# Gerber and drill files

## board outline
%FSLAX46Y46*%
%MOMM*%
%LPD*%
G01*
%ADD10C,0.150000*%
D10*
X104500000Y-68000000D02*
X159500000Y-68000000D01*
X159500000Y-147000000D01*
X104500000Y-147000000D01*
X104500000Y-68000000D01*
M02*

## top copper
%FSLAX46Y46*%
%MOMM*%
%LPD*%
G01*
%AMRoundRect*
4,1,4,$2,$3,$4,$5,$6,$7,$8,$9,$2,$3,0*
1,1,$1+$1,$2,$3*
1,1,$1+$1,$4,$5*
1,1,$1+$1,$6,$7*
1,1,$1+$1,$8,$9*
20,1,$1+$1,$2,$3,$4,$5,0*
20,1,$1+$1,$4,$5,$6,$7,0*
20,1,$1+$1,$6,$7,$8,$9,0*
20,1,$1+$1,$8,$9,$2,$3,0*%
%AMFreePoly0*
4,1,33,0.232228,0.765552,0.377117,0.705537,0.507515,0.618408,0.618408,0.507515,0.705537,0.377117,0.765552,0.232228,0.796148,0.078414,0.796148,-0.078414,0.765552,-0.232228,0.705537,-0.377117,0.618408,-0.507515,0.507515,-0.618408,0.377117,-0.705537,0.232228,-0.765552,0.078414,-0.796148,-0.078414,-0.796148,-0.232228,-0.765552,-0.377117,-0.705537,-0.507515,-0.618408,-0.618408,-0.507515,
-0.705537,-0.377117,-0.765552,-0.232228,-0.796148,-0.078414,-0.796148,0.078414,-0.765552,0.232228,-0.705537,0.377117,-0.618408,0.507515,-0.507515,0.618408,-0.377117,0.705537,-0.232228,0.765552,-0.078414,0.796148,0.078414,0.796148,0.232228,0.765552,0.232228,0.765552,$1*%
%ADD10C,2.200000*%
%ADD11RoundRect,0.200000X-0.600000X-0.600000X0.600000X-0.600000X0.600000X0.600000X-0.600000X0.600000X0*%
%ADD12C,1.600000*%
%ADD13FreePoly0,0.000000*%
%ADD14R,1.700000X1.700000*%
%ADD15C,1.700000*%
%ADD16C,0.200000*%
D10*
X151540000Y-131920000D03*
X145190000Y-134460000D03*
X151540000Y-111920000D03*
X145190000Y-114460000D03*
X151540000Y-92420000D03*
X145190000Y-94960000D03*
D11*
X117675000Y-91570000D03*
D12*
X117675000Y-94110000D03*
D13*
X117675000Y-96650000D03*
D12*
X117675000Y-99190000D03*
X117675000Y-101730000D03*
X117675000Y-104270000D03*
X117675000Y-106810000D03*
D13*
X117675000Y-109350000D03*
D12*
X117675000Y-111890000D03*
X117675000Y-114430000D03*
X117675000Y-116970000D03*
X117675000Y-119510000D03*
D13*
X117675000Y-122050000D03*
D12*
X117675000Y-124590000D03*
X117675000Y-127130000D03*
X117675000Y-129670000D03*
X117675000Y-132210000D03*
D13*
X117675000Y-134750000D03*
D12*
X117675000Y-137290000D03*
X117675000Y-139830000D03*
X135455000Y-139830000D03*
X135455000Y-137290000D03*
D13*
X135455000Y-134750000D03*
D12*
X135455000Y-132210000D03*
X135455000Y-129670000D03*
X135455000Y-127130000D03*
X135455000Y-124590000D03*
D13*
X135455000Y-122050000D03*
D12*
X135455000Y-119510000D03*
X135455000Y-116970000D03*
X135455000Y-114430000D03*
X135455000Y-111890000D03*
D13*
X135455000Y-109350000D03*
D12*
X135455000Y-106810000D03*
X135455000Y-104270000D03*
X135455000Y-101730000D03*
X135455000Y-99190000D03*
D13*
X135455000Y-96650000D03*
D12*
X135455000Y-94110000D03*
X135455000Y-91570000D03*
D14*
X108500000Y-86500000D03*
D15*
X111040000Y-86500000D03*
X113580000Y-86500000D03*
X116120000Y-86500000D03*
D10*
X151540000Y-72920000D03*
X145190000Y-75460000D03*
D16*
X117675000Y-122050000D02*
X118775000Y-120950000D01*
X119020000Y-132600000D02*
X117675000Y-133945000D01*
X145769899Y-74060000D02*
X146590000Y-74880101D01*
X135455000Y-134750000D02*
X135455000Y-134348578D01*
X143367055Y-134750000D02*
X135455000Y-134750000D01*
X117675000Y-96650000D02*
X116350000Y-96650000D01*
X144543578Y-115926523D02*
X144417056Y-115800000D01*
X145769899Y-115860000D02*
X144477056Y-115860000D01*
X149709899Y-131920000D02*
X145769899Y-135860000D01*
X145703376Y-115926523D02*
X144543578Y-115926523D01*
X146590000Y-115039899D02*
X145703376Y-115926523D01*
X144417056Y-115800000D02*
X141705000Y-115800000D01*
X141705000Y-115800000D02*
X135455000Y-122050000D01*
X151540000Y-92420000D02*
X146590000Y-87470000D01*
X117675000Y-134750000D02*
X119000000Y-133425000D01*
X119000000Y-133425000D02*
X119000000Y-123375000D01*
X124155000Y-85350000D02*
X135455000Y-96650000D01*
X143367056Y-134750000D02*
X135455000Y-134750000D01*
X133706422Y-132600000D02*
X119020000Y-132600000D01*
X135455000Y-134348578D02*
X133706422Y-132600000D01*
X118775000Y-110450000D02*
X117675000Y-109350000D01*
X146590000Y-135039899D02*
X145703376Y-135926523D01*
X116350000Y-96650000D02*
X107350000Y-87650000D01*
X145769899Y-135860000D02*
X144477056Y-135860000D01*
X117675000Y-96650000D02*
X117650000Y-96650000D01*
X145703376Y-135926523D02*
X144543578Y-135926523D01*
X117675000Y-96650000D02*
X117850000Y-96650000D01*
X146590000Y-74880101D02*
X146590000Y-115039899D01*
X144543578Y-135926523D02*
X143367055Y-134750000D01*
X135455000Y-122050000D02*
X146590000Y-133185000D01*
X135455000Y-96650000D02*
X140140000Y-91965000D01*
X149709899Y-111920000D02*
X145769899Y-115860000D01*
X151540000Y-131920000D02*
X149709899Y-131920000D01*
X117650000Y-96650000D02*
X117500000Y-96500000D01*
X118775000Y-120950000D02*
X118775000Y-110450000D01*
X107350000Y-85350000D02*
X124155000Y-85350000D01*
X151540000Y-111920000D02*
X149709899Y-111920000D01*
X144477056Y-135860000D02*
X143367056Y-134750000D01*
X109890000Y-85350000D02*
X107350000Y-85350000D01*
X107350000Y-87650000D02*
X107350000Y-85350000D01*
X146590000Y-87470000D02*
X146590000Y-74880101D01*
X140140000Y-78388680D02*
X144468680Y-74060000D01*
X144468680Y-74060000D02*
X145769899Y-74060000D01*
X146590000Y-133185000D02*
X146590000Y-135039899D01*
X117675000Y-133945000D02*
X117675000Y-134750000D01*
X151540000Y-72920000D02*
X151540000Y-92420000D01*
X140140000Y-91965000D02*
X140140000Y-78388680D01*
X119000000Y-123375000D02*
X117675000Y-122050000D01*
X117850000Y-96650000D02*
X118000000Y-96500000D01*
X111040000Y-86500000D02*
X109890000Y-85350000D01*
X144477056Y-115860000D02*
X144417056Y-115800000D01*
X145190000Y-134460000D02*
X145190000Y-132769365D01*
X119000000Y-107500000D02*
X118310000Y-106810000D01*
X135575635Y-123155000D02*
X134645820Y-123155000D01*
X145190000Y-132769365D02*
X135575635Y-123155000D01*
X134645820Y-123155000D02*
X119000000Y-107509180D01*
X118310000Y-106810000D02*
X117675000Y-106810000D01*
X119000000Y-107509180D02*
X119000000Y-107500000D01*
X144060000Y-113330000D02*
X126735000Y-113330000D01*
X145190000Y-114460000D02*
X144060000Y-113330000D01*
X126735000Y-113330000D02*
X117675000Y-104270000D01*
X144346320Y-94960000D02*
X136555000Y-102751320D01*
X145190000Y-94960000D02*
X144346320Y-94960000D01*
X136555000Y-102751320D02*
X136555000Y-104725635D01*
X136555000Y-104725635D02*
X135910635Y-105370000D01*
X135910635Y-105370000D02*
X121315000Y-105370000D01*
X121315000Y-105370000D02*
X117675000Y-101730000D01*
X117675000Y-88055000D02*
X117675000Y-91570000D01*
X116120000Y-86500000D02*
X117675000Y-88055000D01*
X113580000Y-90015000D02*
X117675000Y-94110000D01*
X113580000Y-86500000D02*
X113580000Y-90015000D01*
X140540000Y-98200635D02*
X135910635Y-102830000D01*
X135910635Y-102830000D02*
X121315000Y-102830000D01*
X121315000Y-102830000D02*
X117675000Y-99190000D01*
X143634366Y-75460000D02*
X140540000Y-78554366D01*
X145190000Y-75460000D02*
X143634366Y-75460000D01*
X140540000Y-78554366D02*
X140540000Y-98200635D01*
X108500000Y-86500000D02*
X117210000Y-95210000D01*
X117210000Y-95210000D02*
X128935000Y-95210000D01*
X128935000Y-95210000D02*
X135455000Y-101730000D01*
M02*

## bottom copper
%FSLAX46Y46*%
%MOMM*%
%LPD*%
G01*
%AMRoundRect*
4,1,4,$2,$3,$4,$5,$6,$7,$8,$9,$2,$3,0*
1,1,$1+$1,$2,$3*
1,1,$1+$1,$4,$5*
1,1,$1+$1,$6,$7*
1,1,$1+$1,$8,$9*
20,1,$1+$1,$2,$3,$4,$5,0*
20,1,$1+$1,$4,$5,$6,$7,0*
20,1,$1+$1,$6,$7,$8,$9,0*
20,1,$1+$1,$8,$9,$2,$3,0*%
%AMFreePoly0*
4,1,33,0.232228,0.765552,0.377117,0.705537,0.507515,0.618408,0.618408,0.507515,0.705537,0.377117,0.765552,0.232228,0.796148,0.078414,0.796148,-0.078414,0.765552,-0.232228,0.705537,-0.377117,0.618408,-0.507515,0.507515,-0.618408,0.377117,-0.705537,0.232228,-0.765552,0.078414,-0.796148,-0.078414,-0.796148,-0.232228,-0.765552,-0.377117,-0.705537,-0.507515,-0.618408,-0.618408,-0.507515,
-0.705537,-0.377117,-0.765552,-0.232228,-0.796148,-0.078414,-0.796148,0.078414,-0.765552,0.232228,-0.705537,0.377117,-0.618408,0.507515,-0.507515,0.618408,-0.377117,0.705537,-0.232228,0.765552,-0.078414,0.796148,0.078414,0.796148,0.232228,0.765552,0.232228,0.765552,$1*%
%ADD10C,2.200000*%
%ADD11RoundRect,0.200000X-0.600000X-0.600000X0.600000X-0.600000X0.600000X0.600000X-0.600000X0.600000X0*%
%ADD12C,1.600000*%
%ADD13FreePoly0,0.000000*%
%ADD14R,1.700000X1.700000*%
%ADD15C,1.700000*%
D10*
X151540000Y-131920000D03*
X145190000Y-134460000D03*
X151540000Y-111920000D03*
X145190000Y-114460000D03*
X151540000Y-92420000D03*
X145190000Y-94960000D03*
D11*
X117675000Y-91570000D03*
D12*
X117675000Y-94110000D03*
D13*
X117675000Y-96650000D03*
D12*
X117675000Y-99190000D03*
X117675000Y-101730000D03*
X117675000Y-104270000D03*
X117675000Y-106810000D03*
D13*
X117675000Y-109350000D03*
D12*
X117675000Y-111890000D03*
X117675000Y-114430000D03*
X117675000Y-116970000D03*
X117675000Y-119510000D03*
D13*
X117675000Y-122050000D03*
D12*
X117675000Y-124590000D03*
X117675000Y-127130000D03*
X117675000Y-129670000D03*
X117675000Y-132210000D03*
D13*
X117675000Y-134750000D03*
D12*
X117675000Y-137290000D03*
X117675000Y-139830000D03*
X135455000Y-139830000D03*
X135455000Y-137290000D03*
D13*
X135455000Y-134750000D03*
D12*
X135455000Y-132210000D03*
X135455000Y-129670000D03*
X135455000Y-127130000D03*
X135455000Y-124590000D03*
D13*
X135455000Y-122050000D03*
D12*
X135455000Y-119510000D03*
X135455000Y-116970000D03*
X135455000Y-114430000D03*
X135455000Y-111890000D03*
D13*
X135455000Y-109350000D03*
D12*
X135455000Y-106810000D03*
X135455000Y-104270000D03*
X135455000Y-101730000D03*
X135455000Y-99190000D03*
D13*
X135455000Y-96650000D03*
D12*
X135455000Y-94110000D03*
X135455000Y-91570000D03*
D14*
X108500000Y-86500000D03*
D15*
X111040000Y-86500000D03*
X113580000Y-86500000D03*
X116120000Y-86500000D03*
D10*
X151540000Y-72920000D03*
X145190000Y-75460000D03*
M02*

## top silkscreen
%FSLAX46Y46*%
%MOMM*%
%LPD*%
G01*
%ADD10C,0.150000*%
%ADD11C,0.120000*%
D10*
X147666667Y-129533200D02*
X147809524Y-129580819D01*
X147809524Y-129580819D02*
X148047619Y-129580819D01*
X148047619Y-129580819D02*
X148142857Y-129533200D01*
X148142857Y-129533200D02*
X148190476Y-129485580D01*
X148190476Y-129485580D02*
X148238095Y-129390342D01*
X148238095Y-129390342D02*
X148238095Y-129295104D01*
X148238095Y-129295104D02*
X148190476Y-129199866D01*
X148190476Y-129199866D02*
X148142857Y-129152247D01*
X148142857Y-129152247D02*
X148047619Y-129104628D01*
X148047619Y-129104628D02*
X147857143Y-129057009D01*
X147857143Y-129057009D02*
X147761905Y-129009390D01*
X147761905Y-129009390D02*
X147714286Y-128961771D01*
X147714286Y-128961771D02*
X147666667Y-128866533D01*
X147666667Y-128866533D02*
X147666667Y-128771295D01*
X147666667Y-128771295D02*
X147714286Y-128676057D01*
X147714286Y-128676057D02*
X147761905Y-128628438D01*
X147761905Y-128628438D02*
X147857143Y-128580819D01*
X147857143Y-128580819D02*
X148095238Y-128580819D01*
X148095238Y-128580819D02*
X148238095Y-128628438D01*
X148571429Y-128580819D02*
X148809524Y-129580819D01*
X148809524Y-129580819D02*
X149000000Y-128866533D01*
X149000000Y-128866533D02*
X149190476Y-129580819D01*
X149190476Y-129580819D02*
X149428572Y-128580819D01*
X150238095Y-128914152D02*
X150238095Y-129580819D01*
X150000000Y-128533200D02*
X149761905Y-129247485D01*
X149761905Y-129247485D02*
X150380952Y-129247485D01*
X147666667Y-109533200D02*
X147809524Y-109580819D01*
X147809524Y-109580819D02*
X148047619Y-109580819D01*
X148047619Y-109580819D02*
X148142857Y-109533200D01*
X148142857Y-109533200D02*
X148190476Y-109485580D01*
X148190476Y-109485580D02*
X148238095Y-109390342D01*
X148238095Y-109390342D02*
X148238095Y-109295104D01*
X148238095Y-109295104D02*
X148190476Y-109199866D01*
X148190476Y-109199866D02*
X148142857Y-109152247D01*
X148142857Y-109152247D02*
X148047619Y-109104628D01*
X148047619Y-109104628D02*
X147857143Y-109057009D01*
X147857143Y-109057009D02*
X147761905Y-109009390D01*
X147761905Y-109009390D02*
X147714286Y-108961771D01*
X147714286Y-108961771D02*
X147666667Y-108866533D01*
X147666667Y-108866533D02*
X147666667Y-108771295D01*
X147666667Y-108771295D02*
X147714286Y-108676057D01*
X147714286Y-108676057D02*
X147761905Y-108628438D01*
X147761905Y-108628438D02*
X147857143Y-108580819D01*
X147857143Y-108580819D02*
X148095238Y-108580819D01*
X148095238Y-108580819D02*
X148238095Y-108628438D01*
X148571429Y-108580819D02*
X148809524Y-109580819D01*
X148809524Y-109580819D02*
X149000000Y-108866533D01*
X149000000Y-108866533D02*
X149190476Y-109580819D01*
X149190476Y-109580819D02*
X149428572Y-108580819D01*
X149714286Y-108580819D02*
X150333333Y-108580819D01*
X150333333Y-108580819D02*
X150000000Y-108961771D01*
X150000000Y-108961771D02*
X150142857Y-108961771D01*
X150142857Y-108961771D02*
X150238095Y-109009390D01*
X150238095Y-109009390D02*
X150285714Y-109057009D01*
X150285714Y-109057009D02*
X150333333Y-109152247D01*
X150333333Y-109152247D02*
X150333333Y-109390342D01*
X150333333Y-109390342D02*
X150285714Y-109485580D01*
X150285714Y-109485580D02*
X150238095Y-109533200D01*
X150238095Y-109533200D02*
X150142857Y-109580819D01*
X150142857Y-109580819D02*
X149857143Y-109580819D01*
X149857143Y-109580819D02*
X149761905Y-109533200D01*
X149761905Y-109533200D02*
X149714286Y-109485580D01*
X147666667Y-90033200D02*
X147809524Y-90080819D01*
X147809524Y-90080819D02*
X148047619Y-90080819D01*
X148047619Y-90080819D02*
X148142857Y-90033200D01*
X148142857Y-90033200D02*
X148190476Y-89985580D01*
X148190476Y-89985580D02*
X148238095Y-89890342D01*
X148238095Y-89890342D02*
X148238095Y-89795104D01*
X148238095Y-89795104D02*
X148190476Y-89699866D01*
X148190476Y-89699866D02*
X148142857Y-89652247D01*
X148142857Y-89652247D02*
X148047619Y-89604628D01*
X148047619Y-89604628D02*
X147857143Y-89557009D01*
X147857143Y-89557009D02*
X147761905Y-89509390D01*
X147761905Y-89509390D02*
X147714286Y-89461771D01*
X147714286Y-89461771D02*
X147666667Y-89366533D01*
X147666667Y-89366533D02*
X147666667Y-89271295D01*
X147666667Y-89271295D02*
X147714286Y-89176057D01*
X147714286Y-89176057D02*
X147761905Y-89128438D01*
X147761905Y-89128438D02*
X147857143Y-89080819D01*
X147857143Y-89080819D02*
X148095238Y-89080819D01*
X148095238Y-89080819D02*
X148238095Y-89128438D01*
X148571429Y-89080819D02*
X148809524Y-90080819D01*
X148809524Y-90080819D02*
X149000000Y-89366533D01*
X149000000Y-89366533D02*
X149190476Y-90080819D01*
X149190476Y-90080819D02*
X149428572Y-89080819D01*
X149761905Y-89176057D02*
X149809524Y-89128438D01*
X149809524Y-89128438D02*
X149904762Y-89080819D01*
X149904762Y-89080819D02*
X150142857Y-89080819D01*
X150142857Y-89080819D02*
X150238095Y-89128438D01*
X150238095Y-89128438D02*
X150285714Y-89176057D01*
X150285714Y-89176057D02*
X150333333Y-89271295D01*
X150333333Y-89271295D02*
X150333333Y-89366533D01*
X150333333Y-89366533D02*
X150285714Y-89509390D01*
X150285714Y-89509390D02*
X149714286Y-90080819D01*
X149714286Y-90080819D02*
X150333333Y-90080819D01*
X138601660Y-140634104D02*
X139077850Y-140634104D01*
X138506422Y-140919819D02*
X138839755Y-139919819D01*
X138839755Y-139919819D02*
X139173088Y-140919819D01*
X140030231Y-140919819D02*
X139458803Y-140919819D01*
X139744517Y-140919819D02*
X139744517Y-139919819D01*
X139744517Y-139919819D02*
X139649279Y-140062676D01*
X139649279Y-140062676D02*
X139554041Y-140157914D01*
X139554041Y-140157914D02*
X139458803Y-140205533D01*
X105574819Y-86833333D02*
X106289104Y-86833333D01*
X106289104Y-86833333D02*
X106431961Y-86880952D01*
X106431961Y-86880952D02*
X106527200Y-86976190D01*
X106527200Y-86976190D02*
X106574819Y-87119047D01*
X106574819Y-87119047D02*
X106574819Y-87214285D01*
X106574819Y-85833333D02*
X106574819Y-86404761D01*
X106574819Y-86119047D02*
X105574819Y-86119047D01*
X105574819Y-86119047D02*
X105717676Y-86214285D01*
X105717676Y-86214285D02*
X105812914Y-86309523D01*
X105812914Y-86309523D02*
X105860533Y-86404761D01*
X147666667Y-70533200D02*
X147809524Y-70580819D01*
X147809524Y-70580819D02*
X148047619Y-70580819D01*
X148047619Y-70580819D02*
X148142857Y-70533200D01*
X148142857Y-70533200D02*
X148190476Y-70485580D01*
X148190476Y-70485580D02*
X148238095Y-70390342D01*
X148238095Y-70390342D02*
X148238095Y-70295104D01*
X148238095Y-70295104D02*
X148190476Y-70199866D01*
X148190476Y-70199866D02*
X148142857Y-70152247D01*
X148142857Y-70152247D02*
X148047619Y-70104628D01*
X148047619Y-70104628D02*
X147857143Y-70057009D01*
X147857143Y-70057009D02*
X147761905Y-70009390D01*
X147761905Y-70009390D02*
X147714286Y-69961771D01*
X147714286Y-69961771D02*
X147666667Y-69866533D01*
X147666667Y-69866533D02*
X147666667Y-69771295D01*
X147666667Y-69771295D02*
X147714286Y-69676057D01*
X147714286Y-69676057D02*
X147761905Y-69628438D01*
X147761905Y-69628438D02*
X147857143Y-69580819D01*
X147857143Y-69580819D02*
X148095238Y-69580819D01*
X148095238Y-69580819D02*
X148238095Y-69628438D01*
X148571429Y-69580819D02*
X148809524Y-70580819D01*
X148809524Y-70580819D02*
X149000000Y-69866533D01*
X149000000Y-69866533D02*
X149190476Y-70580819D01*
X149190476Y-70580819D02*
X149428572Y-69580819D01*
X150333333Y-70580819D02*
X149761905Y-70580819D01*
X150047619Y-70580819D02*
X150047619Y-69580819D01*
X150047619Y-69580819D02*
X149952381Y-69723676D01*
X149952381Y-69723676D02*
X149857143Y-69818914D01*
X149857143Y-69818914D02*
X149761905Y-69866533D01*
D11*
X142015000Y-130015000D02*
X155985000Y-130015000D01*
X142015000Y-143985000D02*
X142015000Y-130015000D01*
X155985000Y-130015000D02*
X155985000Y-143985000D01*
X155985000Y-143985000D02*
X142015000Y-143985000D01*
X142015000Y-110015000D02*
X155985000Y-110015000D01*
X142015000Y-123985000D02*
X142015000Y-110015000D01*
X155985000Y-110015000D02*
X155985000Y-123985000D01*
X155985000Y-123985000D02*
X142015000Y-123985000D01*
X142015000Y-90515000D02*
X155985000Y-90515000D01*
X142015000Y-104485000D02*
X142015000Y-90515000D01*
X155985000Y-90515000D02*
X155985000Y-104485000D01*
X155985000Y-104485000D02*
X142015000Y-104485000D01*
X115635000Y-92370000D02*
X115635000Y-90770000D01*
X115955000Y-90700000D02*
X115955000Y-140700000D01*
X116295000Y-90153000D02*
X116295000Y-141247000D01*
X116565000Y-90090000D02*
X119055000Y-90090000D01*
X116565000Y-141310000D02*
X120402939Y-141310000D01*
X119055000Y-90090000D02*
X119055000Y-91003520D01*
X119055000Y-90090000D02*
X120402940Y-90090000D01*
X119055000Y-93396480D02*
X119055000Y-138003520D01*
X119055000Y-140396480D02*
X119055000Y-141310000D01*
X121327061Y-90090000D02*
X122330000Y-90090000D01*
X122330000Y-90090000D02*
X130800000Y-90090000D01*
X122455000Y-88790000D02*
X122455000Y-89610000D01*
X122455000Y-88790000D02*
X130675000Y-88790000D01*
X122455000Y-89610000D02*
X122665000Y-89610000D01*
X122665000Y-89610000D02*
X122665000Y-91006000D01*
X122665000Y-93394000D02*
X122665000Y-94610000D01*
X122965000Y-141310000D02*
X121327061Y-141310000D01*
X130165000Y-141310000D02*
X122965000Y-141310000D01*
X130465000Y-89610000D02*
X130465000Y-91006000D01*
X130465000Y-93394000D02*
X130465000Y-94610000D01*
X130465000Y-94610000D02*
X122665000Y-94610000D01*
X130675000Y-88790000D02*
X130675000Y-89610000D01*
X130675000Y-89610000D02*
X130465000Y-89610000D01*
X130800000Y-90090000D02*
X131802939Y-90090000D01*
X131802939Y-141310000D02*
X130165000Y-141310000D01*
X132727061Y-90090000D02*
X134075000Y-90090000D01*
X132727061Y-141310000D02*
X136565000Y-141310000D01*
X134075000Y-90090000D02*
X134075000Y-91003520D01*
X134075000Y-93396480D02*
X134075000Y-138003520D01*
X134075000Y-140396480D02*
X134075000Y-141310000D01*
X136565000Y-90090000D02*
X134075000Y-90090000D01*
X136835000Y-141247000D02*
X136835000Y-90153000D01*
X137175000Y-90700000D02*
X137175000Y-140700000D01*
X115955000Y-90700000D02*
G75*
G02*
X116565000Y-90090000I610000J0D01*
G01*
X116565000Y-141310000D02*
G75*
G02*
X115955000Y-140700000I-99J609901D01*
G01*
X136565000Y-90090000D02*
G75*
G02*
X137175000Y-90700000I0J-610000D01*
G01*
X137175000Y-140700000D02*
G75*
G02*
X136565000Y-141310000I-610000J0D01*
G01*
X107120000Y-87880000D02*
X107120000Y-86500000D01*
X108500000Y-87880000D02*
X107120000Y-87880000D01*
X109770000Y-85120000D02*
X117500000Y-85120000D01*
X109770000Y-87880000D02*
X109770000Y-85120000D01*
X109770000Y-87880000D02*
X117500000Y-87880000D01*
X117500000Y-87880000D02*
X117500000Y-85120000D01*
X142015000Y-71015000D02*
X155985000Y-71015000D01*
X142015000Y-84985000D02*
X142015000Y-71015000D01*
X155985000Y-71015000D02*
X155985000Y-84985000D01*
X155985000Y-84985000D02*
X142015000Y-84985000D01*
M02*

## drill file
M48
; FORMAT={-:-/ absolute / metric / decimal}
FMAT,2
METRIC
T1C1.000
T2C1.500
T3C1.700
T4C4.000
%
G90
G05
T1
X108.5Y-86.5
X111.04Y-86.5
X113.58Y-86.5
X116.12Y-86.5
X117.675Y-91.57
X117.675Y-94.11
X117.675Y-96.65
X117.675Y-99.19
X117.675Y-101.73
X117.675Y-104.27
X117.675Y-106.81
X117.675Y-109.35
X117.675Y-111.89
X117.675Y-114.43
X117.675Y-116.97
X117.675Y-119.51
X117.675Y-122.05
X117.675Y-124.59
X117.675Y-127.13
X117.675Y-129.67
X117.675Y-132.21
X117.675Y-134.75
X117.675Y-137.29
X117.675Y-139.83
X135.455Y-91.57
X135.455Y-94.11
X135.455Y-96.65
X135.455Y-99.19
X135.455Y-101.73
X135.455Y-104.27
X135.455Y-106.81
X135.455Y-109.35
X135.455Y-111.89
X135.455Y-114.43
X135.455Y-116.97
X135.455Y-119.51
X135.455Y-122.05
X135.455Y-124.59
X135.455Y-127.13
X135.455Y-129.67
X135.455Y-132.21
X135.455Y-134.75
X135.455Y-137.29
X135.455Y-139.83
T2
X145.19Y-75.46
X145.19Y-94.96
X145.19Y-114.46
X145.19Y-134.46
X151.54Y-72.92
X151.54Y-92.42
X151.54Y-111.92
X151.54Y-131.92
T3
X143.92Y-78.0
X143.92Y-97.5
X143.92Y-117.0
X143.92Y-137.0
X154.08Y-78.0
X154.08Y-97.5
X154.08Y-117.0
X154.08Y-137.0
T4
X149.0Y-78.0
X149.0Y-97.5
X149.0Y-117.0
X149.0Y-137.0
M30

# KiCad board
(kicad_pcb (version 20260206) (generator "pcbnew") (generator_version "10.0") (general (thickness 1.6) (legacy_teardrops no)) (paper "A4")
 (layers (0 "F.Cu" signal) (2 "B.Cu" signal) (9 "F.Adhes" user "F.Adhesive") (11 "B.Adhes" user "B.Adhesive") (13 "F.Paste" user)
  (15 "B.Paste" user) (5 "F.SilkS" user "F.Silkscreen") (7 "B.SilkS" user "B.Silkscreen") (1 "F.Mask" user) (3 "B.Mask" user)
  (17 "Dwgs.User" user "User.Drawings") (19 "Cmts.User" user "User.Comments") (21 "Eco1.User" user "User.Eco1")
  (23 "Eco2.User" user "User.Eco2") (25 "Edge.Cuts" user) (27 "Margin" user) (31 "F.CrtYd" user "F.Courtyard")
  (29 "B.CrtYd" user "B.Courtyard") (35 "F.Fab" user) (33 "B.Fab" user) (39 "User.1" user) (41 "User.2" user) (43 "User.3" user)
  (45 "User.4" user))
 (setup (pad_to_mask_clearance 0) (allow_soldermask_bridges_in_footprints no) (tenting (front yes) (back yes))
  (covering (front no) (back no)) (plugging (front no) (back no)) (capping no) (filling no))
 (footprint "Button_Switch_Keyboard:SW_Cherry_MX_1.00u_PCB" (layer "F.Cu") (at 151.54 131.92)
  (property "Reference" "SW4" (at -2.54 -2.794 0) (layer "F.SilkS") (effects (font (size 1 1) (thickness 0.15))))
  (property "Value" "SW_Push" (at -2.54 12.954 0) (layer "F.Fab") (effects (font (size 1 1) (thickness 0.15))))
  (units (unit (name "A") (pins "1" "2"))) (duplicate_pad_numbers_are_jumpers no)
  (fp_line (start -9.525 -1.905) (end 4.445 -1.905) (stroke (width 0.12) (type solid)) (layer "F.SilkS"))
  (fp_line (start -9.525 12.065) (end -9.525 -1.905) (stroke (width 0.12) (type solid)) (layer "F.SilkS"))
  (fp_line (start 4.445 -1.905) (end 4.445 12.065) (stroke (width 0.12) (type solid)) (layer "F.SilkS"))
  (fp_line (start 4.445 12.065) (end -9.525 12.065) (stroke (width 0.12) (type solid)) (layer "F.SilkS"))
  (pad "" np_thru_hole circle (at -7.62 5.08) (size 1.7 1.7) (drill 1.7) (layers "*.Cu" "*.Mask"))
  (pad "" np_thru_hole circle (at -2.54 5.08) (size 4 4) (drill 4) (layers "*.Cu" "*.Mask"))
  (pad "" np_thru_hole circle (at 2.54 5.08) (size 1.7 1.7) (drill 1.7) (layers "*.Cu" "*.Mask"))
  (pad "1" thru_hole circle (at 0 0) (size 2.2 2.2) (drill 1.5) (layers "*.Cu" "*.Mask") (remove_unused_layers no) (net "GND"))
  (pad "2" thru_hole circle (at -6.35 2.54) (size 2.2 2.2) (drill 1.5) (layers "*.Cu" "*.Mask") (remove_unused_layers no)
   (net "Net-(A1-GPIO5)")))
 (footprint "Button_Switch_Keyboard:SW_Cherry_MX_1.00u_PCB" (layer "F.Cu") (at 151.54 111.92)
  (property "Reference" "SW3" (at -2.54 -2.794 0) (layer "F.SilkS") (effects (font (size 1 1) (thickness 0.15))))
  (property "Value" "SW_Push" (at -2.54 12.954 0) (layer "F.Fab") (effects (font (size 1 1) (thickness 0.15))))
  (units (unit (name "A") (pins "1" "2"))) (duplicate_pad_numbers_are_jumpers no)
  (fp_line (start -9.525 -1.905) (end 4.445 -1.905) (stroke (width 0.12) (type solid)) (layer "F.SilkS"))
  (fp_line (start -9.525 12.065) (end -9.525 -1.905) (stroke (width 0.12) (type solid)) (layer "F.SilkS"))
  (fp_line (start 4.445 -1.905) (end 4.445 12.065) (stroke (width 0.12) (type solid)) (layer "F.SilkS"))
  (fp_line (start 4.445 12.065) (end -9.525 12.065) (stroke (width 0.12) (type solid)) (layer "F.SilkS"))
  (pad "" np_thru_hole circle (at -7.62 5.08) (size 1.7 1.7) (drill 1.7) (layers "*.Cu" "*.Mask"))
  (pad "" np_thru_hole circle (at -2.54 5.08) (size 4 4) (drill 4) (layers "*.Cu" "*.Mask"))
  (pad "" np_thru_hole circle (at 2.54 5.08) (size 1.7 1.7) (drill 1.7) (layers "*.Cu" "*.Mask"))
  (pad "1" thru_hole circle (at 0 0) (size 2.2 2.2) (drill 1.5) (layers "*.Cu" "*.Mask") (remove_unused_layers no) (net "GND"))
  (pad "2" thru_hole circle (at -6.35 2.54) (size 2.2 2.2) (drill 1.5) (layers "*.Cu" "*.Mask") (remove_unused_layers no)
   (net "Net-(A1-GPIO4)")))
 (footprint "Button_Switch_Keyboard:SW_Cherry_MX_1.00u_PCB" (layer "F.Cu") (at 151.54 92.42)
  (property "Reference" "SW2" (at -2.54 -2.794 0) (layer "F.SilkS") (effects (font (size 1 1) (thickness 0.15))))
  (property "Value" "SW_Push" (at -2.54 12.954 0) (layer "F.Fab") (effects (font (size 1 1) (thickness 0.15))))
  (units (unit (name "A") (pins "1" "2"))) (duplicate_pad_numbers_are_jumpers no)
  (fp_line (start -9.525 -1.905) (end 4.445 -1.905) (stroke (width 0.12) (type solid)) (layer "F.SilkS"))
  (fp_line (start -9.525 12.065) (end -9.525 -1.905) (stroke (width 0.12) (type solid)) (layer "F.SilkS"))
  (fp_line (start 4.445 -1.905) (end 4.445 12.065) (stroke (width 0.12) (type solid)) (layer "F.SilkS"))
  (fp_line (start 4.445 12.065) (end -9.525 12.065) (stroke (width 0.12) (type solid)) (layer "F.SilkS"))
  (pad "" np_thru_hole circle (at -7.62 5.08) (size 1.7 1.7) (drill 1.7) (layers "*.Cu" "*.Mask"))
  (pad "" np_thru_hole circle (at -2.54 5.08) (size 4 4) (drill 4) (layers "*.Cu" "*.Mask"))
  (pad "" np_thru_hole circle (at 2.54 5.08) (size 1.7 1.7) (drill 1.7) (layers "*.Cu" "*.Mask"))
  (pad "1" thru_hole circle (at 0 0) (size 2.2 2.2) (drill 1.5) (layers "*.Cu" "*.Mask") (remove_unused_layers no) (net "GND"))
  (pad "2" thru_hole circle (at -6.35 2.54) (size 2.2 2.2) (drill 1.5) (layers "*.Cu" "*.Mask") (remove_unused_layers no)
   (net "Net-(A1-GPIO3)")))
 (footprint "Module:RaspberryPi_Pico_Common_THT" (layer "F.Cu") (at 117.675 91.57)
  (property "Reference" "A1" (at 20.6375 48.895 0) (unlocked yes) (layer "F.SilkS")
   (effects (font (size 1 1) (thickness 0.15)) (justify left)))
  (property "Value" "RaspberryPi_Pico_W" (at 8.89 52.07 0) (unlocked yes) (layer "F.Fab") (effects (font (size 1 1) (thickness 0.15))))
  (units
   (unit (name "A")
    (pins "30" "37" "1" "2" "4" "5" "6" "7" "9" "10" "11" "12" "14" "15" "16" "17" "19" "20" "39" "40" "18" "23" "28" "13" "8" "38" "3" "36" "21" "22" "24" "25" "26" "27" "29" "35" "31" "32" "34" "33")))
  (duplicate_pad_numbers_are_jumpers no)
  (fp_line (start -2.04 0.8) (end -2.04 -0.8) (stroke (width 0.12) (type solid)) (layer "F.SilkS"))
  (fp_line (start -1.72 -0.87) (end -1.72 49.13) (stroke (width 0.12) (type solid)) (layer "F.SilkS"))
  (fp_line (start -1.38 -1.417) (end -1.38 49.677) (stroke (width 0.12) (type solid)) (layer "F.SilkS"))
  (fp_line (start -1.11 -1.48) (end 1.38 -1.48) (stroke (width 0.12) (type solid)) (layer "F.SilkS"))
  (fp_line (start -1.11 49.74) (end 2.727939 49.74) (stroke (width 0.12) (type solid)) (layer "F.SilkS"))
  (fp_line (start 1.38 -1.48) (end 1.38 -0.56648) (stroke (width 0.12) (type solid)) (layer "F.SilkS"))
  (fp_line (start 1.38 -1.48) (end 2.72794 -1.48) (stroke (width 0.12) (type solid)) (layer "F.SilkS"))
  (fp_line (start 1.38 1.82648) (end 1.38 46.43352) (stroke (width 0.12) (type solid)) (layer "F.SilkS"))
  (fp_line (start 1.38 48.82648) (end 1.38 49.74) (stroke (width 0.12) (type solid)) (layer "F.SilkS"))
  (fp_line (start 3.652061 -1.48) (end 4.655 -1.48) (stroke (width 0.12) (type solid)) (layer "F.SilkS"))
  (fp_line (start 4.655 -1.48) (end 13.125 -1.48) (stroke (width 0.12) (type solid)) (layer "F.SilkS"))
  (fp_line (start 4.78 -2.78) (end 4.78 -1.96) (stroke (width 0.12) (type solid)) (layer "F.SilkS"))
  (fp_line (start 4.78 -2.78) (end 13 -2.78) (stroke (width 0.12) (type solid)) (layer "F.SilkS"))
  (fp_line (start 4.78 -1.96) (end 4.99 -1.96) (stroke (width 0.12) (type solid)) (layer "F.SilkS"))
  (fp_line (start 4.99 -1.96) (end 4.99 -0.564) (stroke (width 0.12) (type solid)) (layer "F.SilkS"))
  (fp_line (start 4.99 1.824) (end 4.99 3.04) (stroke (width 0.12) (type solid)) (layer "F.SilkS"))
  (fp_line (start 5.29 49.74) (end 3.652061 49.74) (stroke (width 0.12) (type solid)) (layer "F.SilkS"))
  (fp_line (start 12.49 49.74) (end 5.29 49.74) (stroke (width 0.12) (type solid)) (layer "F.SilkS"))
  (fp_line (start 12.79 -1.96) (end 12.79 -0.564) (stroke (width 0.12) (type solid)) (layer "F.SilkS"))
  (fp_line (start 12.79 1.824) (end 12.79 3.04) (stroke (width 0.12) (type solid)) (layer "F.SilkS"))
  (fp_line (start 12.79 3.04) (end 4.99 3.04) (stroke (width 0.12) (type solid)) (layer "F.SilkS"))
  (fp_line (start 13 -2.78) (end 13 -1.96) (stroke (width 0.12) (type solid)) (layer "F.SilkS"))
  (fp_line (start 13 -1.96) (end 12.79 -1.96) (stroke (width 0.12) (type solid)) (layer "F.SilkS"))
  (fp_line (start 13.125 -1.48) (end 14.127939 -1.48) (stroke (width 0.12) (type solid)) (layer "F.SilkS"))
  (fp_line (start 14.127939 49.74) (end 12.49 49.74) (stroke (width 0.12) (type solid)) (layer "F.SilkS"))
  (fp_line (start 15.052061 -1.48) (end 16.4 -1.48) (stroke (width 0.12) (type solid)) (layer "F.SilkS"))
  (fp_line (start 15.052061 49.74) (end 18.89 49.74) (stroke (width 0.12) (type solid)) (layer "F.SilkS"))
  (fp_line (start 16.4 -1.48) (end 16.4 -0.56648) (stroke (width 0.12) (type solid)) (layer "F.SilkS"))
  (fp_line (start 16.4 1.82648) (end 16.4 46.43352) (stroke (width 0.12) (type solid)) (layer "F.SilkS"))
  (fp_line (start 16.4 48.82648) (end 16.4 49.74) (stroke (width 0.12) (type solid)) (layer "F.SilkS"))
  (fp_line (start 18.89 -1.48) (end 16.4 -1.48) (stroke (width 0.12) (type solid)) (layer "F.SilkS"))
  (fp_line (start 19.16 49.677) (end 19.16 -1.417) (stroke (width 0.12) (type solid)) (layer "F.SilkS"))
  (fp_line (start 19.5 -0.87) (end 19.5 49.13) (stroke (width 0.12) (type solid)) (layer "F.SilkS"))
  (fp_arc (start -1.72 -0.87) (mid -1.541335 -1.301335) (end -1.11 -1.48) (stroke (width 0.12) (type solid)) (layer "F.SilkS"))
  (fp_arc (start -1.11 49.74) (mid -1.541364 49.561364) (end -1.72 49.13) (stroke (width 0.12) (type solid)) (layer "F.SilkS"))
  (fp_arc (start 18.89 -1.48) (mid 19.321335 -1.301335) (end 19.5 -0.87) (stroke (width 0.12) (type solid)) (layer "F.SilkS"))
  (fp_arc (start 19.5 49.13) (mid 19.321335 49.561335) (end 18.89 49.74) (stroke (width 0.12) (type solid)) (layer "F.SilkS"))
  (pad "1" thru_hole roundrect (at 0 0) (size 1.6 1.6) (drill 1) (layers "*.Cu" "*.Mask") (remove_unused_layers no) (roundrect_rratio 0.125)
   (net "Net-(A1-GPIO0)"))
  (pad "2" thru_hole circle (at 0 2.54) (size 1.6 1.6) (drill 1) (layers "*.Cu" "*.Mask") (remove_unused_layers no) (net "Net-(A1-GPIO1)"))
  (pad "3" thru_hole custom (at 0 5.08) (size 1.6 1.6) (drill 1) (layers "*.Cu" "*.Mask") (remove_unused_layers no) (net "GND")
   (options (clearance outline) (anchor circle)) (primitives))
  (pad "4" thru_hole circle (at 0 7.62) (size 1.6 1.6) (drill 1) (layers "*.Cu" "*.Mask") (remove_unused_layers no) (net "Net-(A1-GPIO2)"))
  (pad "5" thru_hole circle (at 0 10.16) (size 1.6 1.6) (drill 1) (layers "*.Cu" "*.Mask") (remove_unused_layers no) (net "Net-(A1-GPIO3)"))
  (pad "6" thru_hole circle (at 0 12.7) (size 1.6 1.6) (drill 1) (layers "*.Cu" "*.Mask") (remove_unused_layers no) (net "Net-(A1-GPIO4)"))
  (pad "7" thru_hole circle (at 0 15.24) (size 1.6 1.6) (drill 1) (layers "*.Cu" "*.Mask") (remove_unused_layers no) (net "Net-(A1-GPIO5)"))
  (pad "8" thru_hole custom (at 0 17.78) (size 1.6 1.6) (drill 1) (layers "*.Cu" "*.Mask") (remove_unused_layers no) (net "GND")
   (options (clearance outline) (anchor circle)) (primitives))
  (pad "9" thru_hole circle (at 0 20.32) (size 1.6 1.6) (drill 1) (layers "*.Cu" "*.Mask") (remove_unused_layers no)
   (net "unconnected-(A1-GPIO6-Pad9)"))
  (pad "10" thru_hole circle (at 0 22.86) (size 1.6 1.6) (drill 1) (layers "*.Cu" "*.Mask") (remove_unused_layers no)
   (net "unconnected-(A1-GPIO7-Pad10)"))
  (pad "11" thru_hole circle (at 0 25.4) (size 1.6 1.6) (drill 1) (layers "*.Cu" "*.Mask") (remove_unused_layers no)
   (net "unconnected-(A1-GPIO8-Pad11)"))
  (pad "12" thru_hole circle (at 0 27.94) (size 1.6 1.6) (drill 1) (layers "*.Cu" "*.Mask") (remove_unused_layers no)
   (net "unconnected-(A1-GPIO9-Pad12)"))
  (pad "13" thru_hole custom (at 0 30.48) (size 1.6 1.6) (drill 1) (layers "*.Cu" "*.Mask") (remove_unused_layers no) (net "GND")
   (options (clearance outline) (anchor circle)) (primitives))
  (pad "14" thru_hole circle (at 0 33.02) (size 1.6 1.6) (drill 1) (layers "*.Cu" "*.Mask") (remove_unused_layers no)
   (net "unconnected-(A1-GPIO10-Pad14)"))
  (pad "15" thru_hole circle (at 0 35.56) (size 1.6 1.6) (drill 1) (layers "*.Cu" "*.Mask") (remove_unused_layers no)
   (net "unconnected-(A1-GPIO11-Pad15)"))
  (pad "16" thru_hole circle (at 0 38.1) (size 1.6 1.6) (drill 1) (layers "*.Cu" "*.Mask") (remove_unused_layers no)
   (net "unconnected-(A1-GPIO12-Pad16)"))
  (pad "17" thru_hole circle (at 0 40.64) (size 1.6 1.6) (drill 1) (layers "*.Cu" "*.Mask") (remove_unused_layers no)
   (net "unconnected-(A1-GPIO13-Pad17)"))
  (pad "18" thru_hole custom (at 0 43.18) (size 1.6 1.6) (drill 1) (layers "*.Cu" "*.Mask") (remove_unused_layers no) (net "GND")
   (options (clearance outline) (anchor circle)) (primitives))
  (pad "19" thru_hole circle (at 0 45.72) (size 1.6 1.6) (drill 1) (layers "*.Cu" "*.Mask") (remove_unused_layers no)
   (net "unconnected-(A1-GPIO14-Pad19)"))
  (pad "20" thru_hole circle (at 0 48.26) (size 1.6 1.6) (drill 1) (layers "*.Cu" "*.Mask") (remove_unused_layers no)
   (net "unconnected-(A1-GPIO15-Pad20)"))
  (pad "21" thru_hole circle (at 17.78 48.26) (size 1.6 1.6) (drill 1) (layers "*.Cu" "*.Mask") (remove_unused_layers no)
   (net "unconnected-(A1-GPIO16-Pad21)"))
  (pad "22" thru_hole circle (at 17.78 45.72) (size 1.6 1.6) (drill 1) (layers "*.Cu" "*.Mask") (remove_unused_layers no)
   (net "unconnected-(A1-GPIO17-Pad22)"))
  (pad "23" thru_hole custom (at 17.78 43.18) (size 1.6 1.6) (drill 1) (layers "*.Cu" "*.Mask") (remove_unused_layers no) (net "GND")
   (options (clearance outline) (anchor circle)) (primitives))
  (pad "24" thru_hole circle (at 17.78 40.64) (size 1.6 1.6) (drill 1) (layers "*.Cu" "*.Mask") (remove_unused_layers no)
   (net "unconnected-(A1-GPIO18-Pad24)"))
  (pad "25" thru_hole circle (at 17.78 38.1) (size 1.6 1.6) (drill 1) (layers "*.Cu" "*.Mask") (remove_unused_layers no)
   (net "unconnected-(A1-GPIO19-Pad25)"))
  (pad "26" thru_hole circle (at 17.78 35.56) (size 1.6 1.6) (drill 1) (layers "*.Cu" "*.Mask") (remove_unused_layers no)
   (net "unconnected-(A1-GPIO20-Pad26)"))
  (pad "27" thru_hole circle (at 17.78 33.02) (size 1.6 1.6) (drill 1) (layers "*.Cu" "*.Mask") (remove_unused_layers no)
   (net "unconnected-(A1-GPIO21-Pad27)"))
  (pad "28" thru_hole custom (at 17.78 30.48) (size 1.6 1.6) (drill 1) (layers "*.Cu" "*.Mask") (remove_unused_layers no) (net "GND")
   (options (clearance outline) (anchor circle)) (primitives))
  (pad "29" thru_hole circle (at 17.78 27.94) (size 1.6 1.6) (drill 1) (layers "*.Cu" "*.Mask") (remove_unused_layers no)
   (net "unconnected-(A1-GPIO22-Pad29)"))
  (pad "30" thru_hole circle (at 17.78 25.4) (size 1.6 1.6) (drill 1) (layers "*.Cu" "*.Mask") (remove_unused_layers no)
   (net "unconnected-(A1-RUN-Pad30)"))
  (pad "31" thru_hole circle (at 17.78 22.86) (size 1.6 1.6) (drill 1) (layers "*.Cu" "*.Mask") (remove_unused_layers no)
   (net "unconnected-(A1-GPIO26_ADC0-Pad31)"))
  (pad "32" thru_hole circle (at 17.78 20.32) (size 1.6 1.6) (drill 1) (layers "*.Cu" "*.Mask") (remove_unused_layers no)
   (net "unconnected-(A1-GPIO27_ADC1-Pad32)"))
  (pad "33" thru_hole custom (at 17.78 17.78) (size 1.6 1.6) (drill 1) (layers "*.Cu" "*.Mask") (remove_unused_layers no)
   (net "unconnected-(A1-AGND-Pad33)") (options (clearance outline) (anchor circle)) (primitives))
  (pad "34" thru_hole circle (at 17.78 15.24) (size 1.6 1.6) (drill 1) (layers "*.Cu" "*.Mask") (remove_unused_layers no)
   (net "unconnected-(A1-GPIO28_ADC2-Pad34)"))
  (pad "35" thru_hole circle (at 17.78 12.7) (size 1.6 1.6) (drill 1) (layers "*.Cu" "*.Mask") (remove_unused_layers no)
   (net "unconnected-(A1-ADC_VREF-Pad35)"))
  (pad "36" thru_hole circle (at 17.78 10.16) (size 1.6 1.6) (drill 1) (layers "*.Cu" "*.Mask") (remove_unused_layers no)
   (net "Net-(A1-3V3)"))
  (pad "37" thru_hole circle (at 17.78 7.62) (size 1.6 1.6) (drill 1) (layers "*.Cu" "*.Mask") (remove_unused_layers no)
   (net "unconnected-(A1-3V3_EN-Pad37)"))
  (pad "38" thru_hole custom (at 17.78 5.08) (size 1.6 1.6) (drill 1) (layers "*.Cu" "*.Mask") (remove_unused_layers no) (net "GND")
   (options (clearance outline) (anchor circle)) (primitives))
  (pad "39" thru_hole circle (at 17.78 2.54) (size 1.6 1.6) (drill 1) (layers "*.Cu" "*.Mask") (remove_unused_layers no)
   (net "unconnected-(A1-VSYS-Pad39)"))
  (pad "40" thru_hole circle (at 17.78 0) (size 1.6 1.6) (drill 1) (layers "*.Cu" "*.Mask") (remove_unused_layers no)
   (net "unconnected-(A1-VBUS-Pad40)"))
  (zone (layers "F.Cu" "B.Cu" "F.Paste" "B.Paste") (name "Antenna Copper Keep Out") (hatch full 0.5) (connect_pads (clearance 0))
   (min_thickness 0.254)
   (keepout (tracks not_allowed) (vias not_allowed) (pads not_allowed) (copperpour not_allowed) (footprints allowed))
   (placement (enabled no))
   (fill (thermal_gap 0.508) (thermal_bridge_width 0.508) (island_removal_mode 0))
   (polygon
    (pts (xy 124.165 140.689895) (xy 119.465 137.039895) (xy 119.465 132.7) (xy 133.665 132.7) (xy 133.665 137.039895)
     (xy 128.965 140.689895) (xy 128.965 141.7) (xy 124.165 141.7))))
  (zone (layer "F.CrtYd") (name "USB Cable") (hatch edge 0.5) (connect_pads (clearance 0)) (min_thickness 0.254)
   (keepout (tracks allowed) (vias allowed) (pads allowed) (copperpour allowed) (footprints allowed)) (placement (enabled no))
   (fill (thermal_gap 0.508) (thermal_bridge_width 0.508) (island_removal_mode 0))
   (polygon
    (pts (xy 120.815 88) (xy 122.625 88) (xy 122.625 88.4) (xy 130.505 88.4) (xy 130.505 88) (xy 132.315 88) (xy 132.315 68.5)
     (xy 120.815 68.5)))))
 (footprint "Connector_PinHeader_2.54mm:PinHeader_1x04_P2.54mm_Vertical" (layer "F.Cu") (at 108.5 86.5 90)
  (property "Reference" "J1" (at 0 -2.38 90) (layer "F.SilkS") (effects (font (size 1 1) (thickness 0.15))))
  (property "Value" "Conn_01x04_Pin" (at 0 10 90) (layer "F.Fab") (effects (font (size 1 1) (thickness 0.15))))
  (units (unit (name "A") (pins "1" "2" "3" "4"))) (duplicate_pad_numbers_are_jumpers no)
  (fp_line (start -1.38 -1.38) (end 0 -1.38) (stroke (width 0.12) (type solid)) (layer "F.SilkS"))
  (fp_line (start -1.38 0) (end -1.38 -1.38) (stroke (width 0.12) (type solid)) (layer "F.SilkS"))
  (fp_line (start 1.38 1.27) (end 1.38 9) (stroke (width 0.12) (type solid)) (layer "F.SilkS"))
  (fp_line (start -1.38 1.27) (end 1.38 1.27) (stroke (width 0.12) (type solid)) (layer "F.SilkS"))
  (fp_line (start -1.38 1.27) (end -1.38 9) (stroke (width 0.12) (type solid)) (layer "F.SilkS"))
  (fp_line (start -1.38 9) (end 1.38 9) (stroke (width 0.12) (type solid)) (layer "F.SilkS"))
  (pad "1" thru_hole rect (at 0 0 90) (size 1.7 1.7) (drill 1) (layers "*.Cu" "*.Mask") (remove_unused_layers no) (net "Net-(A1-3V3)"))
  (pad "2" thru_hole circle (at 0 2.54 90) (size 1.7 1.7) (drill 1) (layers "*.Cu" "*.Mask") (remove_unused_layers no) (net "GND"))
  (pad "3" thru_hole circle (at 0 5.08 90) (size 1.7 1.7) (drill 1) (layers "*.Cu" "*.Mask") (remove_unused_layers no)
   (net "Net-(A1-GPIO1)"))
  (pad "4" thru_hole circle (at 0 7.62 90) (size 1.7 1.7) (drill 1) (layers "*.Cu" "*.Mask") (remove_unused_layers no)
   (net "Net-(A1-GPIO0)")))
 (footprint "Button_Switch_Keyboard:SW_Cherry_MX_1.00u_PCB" (layer "F.Cu") (at 151.54 72.92)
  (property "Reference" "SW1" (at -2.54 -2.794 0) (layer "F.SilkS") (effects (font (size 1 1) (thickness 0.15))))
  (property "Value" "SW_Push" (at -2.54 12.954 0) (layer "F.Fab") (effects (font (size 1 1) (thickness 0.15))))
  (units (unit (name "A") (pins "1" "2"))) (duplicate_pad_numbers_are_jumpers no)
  (fp_line (start -9.525 -1.905) (end 4.445 -1.905) (stroke (width 0.12) (type solid)) (layer "F.SilkS"))
  (fp_line (start -9.525 12.065) (end -9.525 -1.905) (stroke (width 0.12) (type solid)) (layer "F.SilkS"))
  (fp_line (start 4.445 -1.905) (end 4.445 12.065) (stroke (width 0.12) (type solid)) (layer "F.SilkS"))
  (fp_line (start 4.445 12.065) (end -9.525 12.065) (stroke (width 0.12) (type solid)) (layer "F.SilkS"))
  (pad "" np_thru_hole circle (at -7.62 5.08) (size 1.7 1.7) (drill 1.7) (layers "*.Cu" "*.Mask"))
  (pad "" np_thru_hole circle (at -2.54 5.08) (size 4 4) (drill 4) (layers "*.Cu" "*.Mask"))
  (pad "" np_thru_hole circle (at 2.54 5.08) (size 1.7 1.7) (drill 1.7) (layers "*.Cu" "*.Mask"))
  (pad "1" thru_hole circle (at 0 0) (size 2.2 2.2) (drill 1.5) (layers "*.Cu" "*.Mask") (remove_unused_layers no) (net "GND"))
  (pad "2" thru_hole circle (at -6.35 2.54) (size 2.2 2.2) (drill 1.5) (layers "*.Cu" "*.Mask") (remove_unused_layers no)
   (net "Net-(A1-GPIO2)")))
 (gr_rect (start 104.5 68) (end 159.5 147) (stroke (width 0.15) (type default)) (fill no) (layer "Edge.Cuts"))
 (segment (start 117.675 122.05) (end 118.775 120.95) (width 0.2) (layer "F.Cu") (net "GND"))
 (segment (start 119.02 132.6) (end 117.675 133.945) (width 0.2) (layer "F.Cu") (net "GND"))
 (segment (start 145.769899 74.06) (end 146.59 74.880101) (width 0.2) (layer "F.Cu") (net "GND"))
 (segment (start 135.455 134.75) (end 135.455 134.348578) (width 0.2) (layer "F.Cu") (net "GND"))
 (segment (start 143.367055 134.75) (end 135.455 134.75) (width 0.2) (layer "F.Cu") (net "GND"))
 (segment (start 117.675 96.65) (end 116.35 96.65) (width 0.2) (layer "F.Cu") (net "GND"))
 (segment (start 144.543578 115.926523) (end 144.417056 115.8) (width 0.2) (layer "F.Cu") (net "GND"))
 (segment (start 145.769899 115.86) (end 144.477056 115.86) (width 0.2) (layer "F.Cu") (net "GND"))
 (segment (start 149.709899 131.92) (end 145.769899 135.86) (width 0.2) (layer "F.Cu") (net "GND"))
 (segment (start 145.703376 115.926523) (end 144.543578 115.926523) (width 0.2) (layer "F.Cu") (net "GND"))
 (segment (start 146.59 115.039899) (end 145.703376 115.926523) (width 0.2) (layer "F.Cu") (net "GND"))
 (segment (start 144.417056 115.8) (end 141.705 115.8) (width 0.2) (layer "F.Cu") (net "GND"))
 (segment (start 141.705 115.8) (end 135.455 122.05) (width 0.2) (layer "F.Cu") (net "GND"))
 (segment (start 151.54 92.42) (end 146.59 87.47) (width 0.2) (layer "F.Cu") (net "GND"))
 (segment (start 117.675 134.75) (end 119 133.425) (width 0.2) (layer "F.Cu") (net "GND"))
 (segment (start 119 133.425) (end 119 123.375) (width 0.2) (layer "F.Cu") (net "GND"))
 (segment (start 124.155 85.35) (end 135.455 96.65) (width 0.2) (layer "F.Cu") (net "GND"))
 (segment (start 143.367056 134.75) (end 135.455 134.75) (width 0.2) (layer "F.Cu") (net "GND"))
 (segment (start 133.706422 132.6) (end 119.02 132.6) (width 0.2) (layer "F.Cu") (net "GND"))
 (segment (start 135.455 134.348578) (end 133.706422 132.6) (width 0.2) (layer "F.Cu") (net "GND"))
 (segment (start 118.775 110.45) (end 117.675 109.35) (width 0.2) (layer "F.Cu") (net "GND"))
 (segment (start 146.59 135.039899) (end 145.703376 135.926523) (width 0.2) (layer "F.Cu") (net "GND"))
 (segment (start 116.35 96.65) (end 107.35 87.65) (width 0.2) (layer "F.Cu") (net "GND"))
 (segment (start 145.769899 135.86) (end 144.477056 135.86) (width 0.2) (layer "F.Cu") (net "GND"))
 (segment (start 117.675 96.65) (end 117.65 96.65) (width 0.2) (layer "F.Cu") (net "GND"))
 (segment (start 145.703376 135.926523) (end 144.543578 135.926523) (width 0.2) (layer "F.Cu") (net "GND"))
 (segment (start 117.675 96.65) (end 117.85 96.65) (width 0.2) (layer "F.Cu") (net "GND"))
 (segment (start 146.59 74.880101) (end 146.59 115.039899) (width 0.2) (layer "F.Cu") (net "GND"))
 (segment (start 144.543578 135.926523) (end 143.367055 134.75) (width 0.2) (layer "F.Cu") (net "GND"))
 (segment (start 135.455 122.05) (end 146.59 133.185) (width 0.2) (layer "F.Cu") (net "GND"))
 (segment (start 135.455 96.65) (end 140.14 91.965) (width 0.2) (layer "F.Cu") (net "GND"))
 (segment (start 149.709899 111.92) (end 145.769899 115.86) (width 0.2) (layer "F.Cu") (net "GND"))
 (segment (start 151.54 131.92) (end 149.709899 131.92) (width 0.2) (layer "F.Cu") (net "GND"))
 (segment (start 117.65 96.65) (end 117.5 96.5) (width 0.2) (layer "F.Cu") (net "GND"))
 (segment (start 118.775 120.95) (end 118.775 110.45) (width 0.2) (layer "F.Cu") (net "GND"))
 (segment (start 107.35 85.35) (end 124.155 85.35) (width 0.2) (layer "F.Cu") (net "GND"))
 (segment (start 151.54 111.92) (end 149.709899 111.92) (width 0.2) (layer "F.Cu") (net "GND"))
 (segment (start 144.477056 135.86) (end 143.367056 134.75) (width 0.2) (layer "F.Cu") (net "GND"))
 (segment (start 109.89 85.35) (end 107.35 85.35) (width 0.2) (layer "F.Cu") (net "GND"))
 (segment (start 107.35 87.65) (end 107.35 85.35) (width 0.2) (layer "F.Cu") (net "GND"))
 (segment (start 146.59 87.47) (end 146.59 74.880101) (width 0.2) (layer "F.Cu") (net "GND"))
 (segment (start 140.14 78.38868) (end 144.46868 74.06) (width 0.2) (layer "F.Cu") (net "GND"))
 (segment (start 144.46868 74.06) (end 145.769899 74.06) (width 0.2) (layer "F.Cu") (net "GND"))
 (segment (start 146.59 133.185) (end 146.59 135.039899) (width 0.2) (layer "F.Cu") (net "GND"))
 (segment (start 117.675 133.945) (end 117.675 134.75) (width 0.2) (layer "F.Cu") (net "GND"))
 (segment (start 151.54 72.92) (end 151.54 92.42) (width 0.2) (layer "F.Cu") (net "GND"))
 (segment (start 140.14 91.965) (end 140.14 78.38868) (width 0.2) (layer "F.Cu") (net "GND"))
 (segment (start 119 123.375) (end 117.675 122.05) (width 0.2) (layer "F.Cu") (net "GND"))
 (segment (start 117.85 96.65) (end 118 96.5) (width 0.2) (layer "F.Cu") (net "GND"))
 (segment (start 111.04 86.5) (end 109.89 85.35) (width 0.2) (layer "F.Cu") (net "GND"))
 (segment (start 144.477056 115.86) (end 144.417056 115.8) (width 0.2) (layer "F.Cu") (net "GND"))
 (segment (start 145.19 134.46) (end 145.19 132.769365) (width 0.2) (layer "F.Cu") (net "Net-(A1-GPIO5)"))
 (segment (start 119 107.5) (end 118.31 106.81) (width 0.2) (layer "F.Cu") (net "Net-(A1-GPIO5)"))
 (segment (start 135.575635 123.155) (end 134.64582 123.155) (width 0.2) (layer "F.Cu") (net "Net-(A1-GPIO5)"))
 (segment (start 145.19 132.769365) (end 135.575635 123.155) (width 0.2) (layer "F.Cu") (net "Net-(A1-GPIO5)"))
 (segment (start 134.64582 123.155) (end 119 107.50918) (width 0.2) (layer "F.Cu") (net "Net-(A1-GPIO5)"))
 (segment (start 118.31 106.81) (end 117.675 106.81) (width 0.2) (layer "F.Cu") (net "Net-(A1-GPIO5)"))
 (segment (start 119 107.50918) (end 119 107.5) (width 0.2) (layer "F.Cu") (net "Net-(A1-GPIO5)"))
 (segment (start 144.06 113.33) (end 126.735 113.33) (width 0.2) (layer "F.Cu") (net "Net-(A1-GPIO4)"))
 (segment (start 145.19 114.46) (end 144.06 113.33) (width 0.2) (layer "F.Cu") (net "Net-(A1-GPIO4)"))
 (segment (start 126.735 113.33) (end 117.675 104.27) (width 0.2) (layer "F.Cu") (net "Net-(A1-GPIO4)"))
 (segment (start 144.34632 94.96) (end 136.555 102.75132) (width 0.2) (layer "F.Cu") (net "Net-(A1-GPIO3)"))
 (segment (start 145.19 94.96) (end 144.34632 94.96) (width 0.2) (layer "F.Cu") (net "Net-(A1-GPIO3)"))
 (segment (start 136.555 102.75132) (end 136.555 104.725635) (width 0.2) (layer "F.Cu") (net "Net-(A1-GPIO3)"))
 (segment (start 136.555 104.725635) (end 135.910635 105.37) (width 0.2) (layer "F.Cu") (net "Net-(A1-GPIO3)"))
 (segment (start 135.910635 105.37) (end 121.315 105.37) (width 0.2) (layer "F.Cu") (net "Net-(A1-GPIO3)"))
 (segment (start 121.315 105.37) (end 117.675 101.73) (width 0.2) (layer "F.Cu") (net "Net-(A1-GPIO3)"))
 (segment (start 117.675 88.055) (end 117.675 91.57) (width 0.2) (layer "F.Cu") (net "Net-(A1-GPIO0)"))
 (segment (start 116.12 86.5) (end 117.675 88.055) (width 0.2) (layer "F.Cu") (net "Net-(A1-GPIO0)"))
 (segment (start 113.58 90.015) (end 117.675 94.11) (width 0.2) (layer "F.Cu") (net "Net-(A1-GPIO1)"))
 (segment (start 113.58 86.5) (end 113.58 90.015) (width 0.2) (layer "F.Cu") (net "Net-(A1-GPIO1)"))
 (segment (start 140.54 98.200635) (end 135.910635 102.83) (width 0.2) (layer "F.Cu") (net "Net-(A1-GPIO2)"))
 (segment (start 135.910635 102.83) (end 121.315 102.83) (width 0.2) (layer "F.Cu") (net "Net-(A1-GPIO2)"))
 (segment (start 121.315 102.83) (end 117.675 99.19) (width 0.2) (layer "F.Cu") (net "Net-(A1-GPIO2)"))
 (segment (start 143.634366 75.46) (end 140.54 78.554366) (width 0.2) (layer "F.Cu") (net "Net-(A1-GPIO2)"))
 (segment (start 145.19 75.46) (end 143.634366 75.46) (width 0.2) (layer "F.Cu") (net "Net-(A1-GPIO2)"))
 (segment (start 140.54 78.554366) (end 140.54 98.200635) (width 0.2) (layer "F.Cu") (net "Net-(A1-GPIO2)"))
 (segment (start 108.5 86.5) (end 117.21 95.21) (width 0.2) (layer "F.Cu") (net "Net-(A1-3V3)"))
 (segment (start 117.21 95.21) (end 128.935 95.21) (width 0.2) (layer "F.Cu") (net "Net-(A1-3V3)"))
 (segment (start 128.935 95.21) (end 135.455 101.73) (width 0.2) (layer "F.Cu") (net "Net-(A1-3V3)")))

